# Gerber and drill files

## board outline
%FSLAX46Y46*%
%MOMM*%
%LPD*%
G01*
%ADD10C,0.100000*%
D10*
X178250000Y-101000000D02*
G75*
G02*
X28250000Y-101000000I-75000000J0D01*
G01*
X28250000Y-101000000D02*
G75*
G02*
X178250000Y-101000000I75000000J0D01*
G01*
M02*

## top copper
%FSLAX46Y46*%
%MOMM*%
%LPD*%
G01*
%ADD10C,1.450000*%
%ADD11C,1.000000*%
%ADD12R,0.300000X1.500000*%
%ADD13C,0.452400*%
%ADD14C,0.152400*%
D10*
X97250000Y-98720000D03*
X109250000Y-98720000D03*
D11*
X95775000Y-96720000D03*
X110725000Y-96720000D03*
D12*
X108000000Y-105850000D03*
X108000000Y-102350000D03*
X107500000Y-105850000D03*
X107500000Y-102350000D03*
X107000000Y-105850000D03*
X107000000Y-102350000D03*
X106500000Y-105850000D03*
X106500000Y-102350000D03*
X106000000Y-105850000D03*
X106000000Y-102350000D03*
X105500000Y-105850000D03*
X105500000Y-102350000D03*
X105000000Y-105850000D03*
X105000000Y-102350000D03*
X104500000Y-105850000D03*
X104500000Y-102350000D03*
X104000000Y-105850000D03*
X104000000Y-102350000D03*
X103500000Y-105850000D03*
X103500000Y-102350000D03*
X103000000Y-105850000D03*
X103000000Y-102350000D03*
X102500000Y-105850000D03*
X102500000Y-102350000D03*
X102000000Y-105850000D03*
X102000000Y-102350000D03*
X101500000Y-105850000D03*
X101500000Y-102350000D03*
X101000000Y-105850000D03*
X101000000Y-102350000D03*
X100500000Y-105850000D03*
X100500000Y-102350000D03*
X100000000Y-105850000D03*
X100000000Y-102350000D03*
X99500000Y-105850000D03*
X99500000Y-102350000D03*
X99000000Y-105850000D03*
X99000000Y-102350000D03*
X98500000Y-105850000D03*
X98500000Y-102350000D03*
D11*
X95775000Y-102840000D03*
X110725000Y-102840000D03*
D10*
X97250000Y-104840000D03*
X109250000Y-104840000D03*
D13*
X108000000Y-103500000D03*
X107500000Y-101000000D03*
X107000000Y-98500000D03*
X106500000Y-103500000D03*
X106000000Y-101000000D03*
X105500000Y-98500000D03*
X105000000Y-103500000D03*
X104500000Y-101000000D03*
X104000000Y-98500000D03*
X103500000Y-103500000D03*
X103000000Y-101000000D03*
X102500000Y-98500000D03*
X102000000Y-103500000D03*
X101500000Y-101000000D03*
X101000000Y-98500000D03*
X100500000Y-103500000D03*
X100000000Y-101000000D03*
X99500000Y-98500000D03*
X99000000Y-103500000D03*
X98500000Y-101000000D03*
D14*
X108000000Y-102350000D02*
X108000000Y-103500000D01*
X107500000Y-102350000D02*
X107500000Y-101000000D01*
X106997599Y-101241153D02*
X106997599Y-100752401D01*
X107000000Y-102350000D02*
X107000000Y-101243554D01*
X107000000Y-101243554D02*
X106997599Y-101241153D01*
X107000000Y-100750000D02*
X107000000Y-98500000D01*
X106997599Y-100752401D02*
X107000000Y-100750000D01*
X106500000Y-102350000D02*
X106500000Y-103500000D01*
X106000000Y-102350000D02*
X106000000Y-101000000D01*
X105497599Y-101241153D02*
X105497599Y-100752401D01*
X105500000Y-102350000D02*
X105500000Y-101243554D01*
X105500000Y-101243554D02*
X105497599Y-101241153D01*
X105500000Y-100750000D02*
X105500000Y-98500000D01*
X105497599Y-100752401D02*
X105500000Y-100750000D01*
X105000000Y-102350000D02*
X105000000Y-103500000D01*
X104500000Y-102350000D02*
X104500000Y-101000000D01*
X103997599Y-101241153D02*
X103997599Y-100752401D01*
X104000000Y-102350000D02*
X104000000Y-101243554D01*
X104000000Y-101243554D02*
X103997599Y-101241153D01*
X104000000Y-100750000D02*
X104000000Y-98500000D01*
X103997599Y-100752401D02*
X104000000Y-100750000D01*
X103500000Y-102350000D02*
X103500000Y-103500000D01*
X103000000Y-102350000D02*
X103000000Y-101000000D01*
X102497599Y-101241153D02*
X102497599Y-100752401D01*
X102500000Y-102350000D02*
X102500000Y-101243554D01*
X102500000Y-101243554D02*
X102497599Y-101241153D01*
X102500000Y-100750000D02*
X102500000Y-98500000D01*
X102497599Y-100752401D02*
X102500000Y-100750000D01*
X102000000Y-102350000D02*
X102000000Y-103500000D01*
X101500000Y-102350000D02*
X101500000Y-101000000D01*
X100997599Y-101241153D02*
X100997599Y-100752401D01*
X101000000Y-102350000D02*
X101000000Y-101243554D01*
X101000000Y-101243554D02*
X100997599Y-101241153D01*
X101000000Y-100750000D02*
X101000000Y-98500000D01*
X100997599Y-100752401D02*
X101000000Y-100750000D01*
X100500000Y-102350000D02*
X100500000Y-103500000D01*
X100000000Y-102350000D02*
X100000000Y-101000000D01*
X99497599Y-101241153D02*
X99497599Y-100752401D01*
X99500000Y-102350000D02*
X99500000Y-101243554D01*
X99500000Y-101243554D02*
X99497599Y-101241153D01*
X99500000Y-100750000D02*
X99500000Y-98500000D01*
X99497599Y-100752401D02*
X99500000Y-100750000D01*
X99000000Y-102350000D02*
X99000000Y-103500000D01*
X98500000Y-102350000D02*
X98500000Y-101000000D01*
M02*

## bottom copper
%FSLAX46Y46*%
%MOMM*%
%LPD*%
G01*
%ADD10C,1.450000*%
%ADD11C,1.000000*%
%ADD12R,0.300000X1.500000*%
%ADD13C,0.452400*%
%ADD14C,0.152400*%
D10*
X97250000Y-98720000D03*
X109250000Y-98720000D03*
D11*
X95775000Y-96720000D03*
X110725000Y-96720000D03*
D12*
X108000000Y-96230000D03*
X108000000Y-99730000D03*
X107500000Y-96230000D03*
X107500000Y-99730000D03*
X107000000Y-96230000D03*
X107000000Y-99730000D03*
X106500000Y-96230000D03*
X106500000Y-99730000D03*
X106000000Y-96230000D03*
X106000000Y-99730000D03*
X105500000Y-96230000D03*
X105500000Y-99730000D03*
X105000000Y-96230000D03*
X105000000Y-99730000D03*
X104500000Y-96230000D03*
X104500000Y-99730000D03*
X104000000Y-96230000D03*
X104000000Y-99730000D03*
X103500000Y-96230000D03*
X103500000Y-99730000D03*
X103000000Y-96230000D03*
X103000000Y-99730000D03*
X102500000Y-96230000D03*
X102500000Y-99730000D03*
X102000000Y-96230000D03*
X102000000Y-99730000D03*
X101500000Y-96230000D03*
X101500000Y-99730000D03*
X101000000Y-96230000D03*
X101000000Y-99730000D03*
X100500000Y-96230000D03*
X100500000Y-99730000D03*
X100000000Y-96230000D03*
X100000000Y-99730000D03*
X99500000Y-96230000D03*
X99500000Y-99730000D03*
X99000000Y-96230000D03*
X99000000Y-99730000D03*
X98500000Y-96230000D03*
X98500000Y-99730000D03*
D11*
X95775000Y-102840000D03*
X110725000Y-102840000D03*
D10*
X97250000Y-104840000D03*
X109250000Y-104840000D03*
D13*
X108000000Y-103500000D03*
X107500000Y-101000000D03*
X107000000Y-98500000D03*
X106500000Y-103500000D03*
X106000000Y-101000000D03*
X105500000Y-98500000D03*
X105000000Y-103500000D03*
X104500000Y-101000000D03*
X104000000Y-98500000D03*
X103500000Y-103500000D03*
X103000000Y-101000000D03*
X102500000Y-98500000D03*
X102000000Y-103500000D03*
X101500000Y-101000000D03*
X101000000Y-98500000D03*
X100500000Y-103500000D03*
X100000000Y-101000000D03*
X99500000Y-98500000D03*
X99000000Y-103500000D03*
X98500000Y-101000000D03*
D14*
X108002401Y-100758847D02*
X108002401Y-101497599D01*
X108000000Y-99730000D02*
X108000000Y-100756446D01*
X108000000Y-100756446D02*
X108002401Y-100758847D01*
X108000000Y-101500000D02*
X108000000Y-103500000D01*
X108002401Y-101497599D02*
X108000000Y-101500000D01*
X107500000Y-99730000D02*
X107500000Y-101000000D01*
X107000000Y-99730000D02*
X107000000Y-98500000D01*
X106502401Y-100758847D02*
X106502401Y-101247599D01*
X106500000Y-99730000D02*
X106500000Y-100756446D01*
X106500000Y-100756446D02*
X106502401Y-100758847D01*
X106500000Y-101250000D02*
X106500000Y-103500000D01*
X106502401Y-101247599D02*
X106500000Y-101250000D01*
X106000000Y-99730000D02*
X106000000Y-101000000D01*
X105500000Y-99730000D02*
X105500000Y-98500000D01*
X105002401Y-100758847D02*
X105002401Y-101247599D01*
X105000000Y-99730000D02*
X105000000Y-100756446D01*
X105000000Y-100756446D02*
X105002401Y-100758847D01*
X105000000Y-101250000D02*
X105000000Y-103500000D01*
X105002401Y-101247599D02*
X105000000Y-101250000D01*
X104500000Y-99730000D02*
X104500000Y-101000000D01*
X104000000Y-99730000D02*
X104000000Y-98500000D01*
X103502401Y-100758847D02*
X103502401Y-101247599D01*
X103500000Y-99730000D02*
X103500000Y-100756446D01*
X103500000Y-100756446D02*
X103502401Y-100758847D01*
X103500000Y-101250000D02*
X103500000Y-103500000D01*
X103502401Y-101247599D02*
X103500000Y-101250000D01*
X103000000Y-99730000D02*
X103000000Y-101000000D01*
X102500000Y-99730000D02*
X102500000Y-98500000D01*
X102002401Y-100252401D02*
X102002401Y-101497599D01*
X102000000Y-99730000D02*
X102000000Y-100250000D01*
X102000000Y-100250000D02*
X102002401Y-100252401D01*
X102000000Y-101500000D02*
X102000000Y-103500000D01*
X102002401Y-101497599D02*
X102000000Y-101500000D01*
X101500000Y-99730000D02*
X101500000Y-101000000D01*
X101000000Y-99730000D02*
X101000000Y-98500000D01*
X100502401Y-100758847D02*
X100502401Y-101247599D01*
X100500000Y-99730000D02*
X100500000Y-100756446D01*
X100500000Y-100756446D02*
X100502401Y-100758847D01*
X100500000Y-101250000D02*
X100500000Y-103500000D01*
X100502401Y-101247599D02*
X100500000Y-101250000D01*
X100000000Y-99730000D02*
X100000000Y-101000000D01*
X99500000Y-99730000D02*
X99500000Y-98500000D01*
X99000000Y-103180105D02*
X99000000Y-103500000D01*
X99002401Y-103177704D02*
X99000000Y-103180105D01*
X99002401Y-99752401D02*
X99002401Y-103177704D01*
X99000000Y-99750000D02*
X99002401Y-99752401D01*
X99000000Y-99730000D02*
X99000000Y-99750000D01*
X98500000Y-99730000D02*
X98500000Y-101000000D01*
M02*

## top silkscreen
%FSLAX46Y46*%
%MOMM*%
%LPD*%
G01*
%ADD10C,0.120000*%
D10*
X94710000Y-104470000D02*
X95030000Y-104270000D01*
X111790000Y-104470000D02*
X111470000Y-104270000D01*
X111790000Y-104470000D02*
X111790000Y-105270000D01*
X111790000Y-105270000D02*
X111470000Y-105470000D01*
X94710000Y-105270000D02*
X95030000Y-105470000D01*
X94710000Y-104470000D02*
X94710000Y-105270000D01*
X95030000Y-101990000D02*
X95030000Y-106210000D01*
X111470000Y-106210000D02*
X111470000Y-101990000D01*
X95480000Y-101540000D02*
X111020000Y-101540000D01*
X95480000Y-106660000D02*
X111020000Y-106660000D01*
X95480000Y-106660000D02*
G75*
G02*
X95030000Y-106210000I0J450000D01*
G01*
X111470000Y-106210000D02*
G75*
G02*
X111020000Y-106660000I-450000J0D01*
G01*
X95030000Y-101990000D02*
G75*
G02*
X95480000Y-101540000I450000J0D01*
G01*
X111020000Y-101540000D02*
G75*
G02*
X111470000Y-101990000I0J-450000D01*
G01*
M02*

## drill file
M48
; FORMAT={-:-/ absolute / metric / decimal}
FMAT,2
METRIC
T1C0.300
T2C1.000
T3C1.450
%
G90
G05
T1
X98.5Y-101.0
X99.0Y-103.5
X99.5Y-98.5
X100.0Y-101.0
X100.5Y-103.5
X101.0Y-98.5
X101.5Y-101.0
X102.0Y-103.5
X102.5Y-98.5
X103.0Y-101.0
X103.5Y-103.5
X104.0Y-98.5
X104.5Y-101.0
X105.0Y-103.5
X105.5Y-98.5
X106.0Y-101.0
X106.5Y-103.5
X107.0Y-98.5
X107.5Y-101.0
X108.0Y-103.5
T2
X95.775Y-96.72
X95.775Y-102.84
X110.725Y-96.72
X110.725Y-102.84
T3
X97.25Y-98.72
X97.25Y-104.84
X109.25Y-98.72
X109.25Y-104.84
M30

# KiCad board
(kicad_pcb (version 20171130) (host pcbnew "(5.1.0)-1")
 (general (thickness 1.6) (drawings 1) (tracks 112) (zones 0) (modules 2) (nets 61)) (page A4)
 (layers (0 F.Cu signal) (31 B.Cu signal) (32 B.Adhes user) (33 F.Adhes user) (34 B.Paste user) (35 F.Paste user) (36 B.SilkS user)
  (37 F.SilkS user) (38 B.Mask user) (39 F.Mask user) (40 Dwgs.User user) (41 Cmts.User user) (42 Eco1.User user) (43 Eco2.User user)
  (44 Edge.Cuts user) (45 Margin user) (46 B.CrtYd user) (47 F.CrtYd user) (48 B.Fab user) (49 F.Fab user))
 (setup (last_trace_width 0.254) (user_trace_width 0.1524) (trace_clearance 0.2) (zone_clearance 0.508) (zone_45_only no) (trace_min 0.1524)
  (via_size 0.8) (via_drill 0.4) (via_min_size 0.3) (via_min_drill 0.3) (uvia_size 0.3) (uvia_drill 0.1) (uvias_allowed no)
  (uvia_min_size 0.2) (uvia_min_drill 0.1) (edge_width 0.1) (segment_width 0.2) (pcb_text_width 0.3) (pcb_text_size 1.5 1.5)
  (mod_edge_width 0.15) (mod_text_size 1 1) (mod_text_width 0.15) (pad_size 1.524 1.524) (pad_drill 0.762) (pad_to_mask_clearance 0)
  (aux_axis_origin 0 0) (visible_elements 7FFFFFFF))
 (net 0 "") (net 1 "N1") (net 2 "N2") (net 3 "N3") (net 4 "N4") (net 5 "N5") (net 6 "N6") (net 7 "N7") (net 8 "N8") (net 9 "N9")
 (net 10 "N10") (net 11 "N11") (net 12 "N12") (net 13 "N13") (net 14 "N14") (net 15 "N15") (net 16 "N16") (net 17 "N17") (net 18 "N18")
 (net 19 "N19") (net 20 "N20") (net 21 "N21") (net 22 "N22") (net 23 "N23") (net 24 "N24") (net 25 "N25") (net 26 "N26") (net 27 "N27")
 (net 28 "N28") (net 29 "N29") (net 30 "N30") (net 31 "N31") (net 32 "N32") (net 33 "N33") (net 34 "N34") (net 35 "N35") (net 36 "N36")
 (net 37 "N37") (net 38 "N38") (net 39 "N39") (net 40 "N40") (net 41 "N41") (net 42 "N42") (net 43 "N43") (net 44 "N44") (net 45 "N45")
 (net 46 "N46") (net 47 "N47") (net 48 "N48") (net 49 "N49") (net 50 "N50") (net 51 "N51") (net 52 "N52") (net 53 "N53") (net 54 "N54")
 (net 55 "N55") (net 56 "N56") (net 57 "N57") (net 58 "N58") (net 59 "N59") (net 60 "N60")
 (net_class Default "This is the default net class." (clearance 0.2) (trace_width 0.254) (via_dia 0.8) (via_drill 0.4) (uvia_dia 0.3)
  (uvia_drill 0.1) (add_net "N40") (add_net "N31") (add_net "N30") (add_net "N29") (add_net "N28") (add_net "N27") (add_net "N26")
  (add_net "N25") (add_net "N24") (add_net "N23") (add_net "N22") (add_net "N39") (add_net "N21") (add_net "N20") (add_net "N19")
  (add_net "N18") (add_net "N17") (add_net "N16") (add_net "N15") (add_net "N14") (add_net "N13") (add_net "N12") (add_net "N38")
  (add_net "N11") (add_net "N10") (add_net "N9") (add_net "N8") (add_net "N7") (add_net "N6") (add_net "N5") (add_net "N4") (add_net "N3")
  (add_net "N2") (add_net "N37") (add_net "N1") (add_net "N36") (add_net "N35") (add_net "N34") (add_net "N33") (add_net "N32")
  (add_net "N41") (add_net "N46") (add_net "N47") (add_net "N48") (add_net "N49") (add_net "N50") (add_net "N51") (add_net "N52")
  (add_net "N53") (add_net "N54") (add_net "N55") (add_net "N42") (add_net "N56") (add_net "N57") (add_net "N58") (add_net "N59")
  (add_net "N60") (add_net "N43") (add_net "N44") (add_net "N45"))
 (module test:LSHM (layer B.Cu) (at 103.25 97.98 180)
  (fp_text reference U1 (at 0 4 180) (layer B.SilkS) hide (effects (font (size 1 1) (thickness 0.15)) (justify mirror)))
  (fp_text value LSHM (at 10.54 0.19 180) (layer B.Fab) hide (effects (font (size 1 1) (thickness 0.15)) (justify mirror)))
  (pad 41 thru_hole circle (at 6 -0.74 180) (size 1.45 1.45) (drill 1.45) (layers *.Cu *.Mask))
  (pad 41 thru_hole circle (at -6 -0.74 180) (size 1.45 1.45) (drill 1.45) (layers *.Cu *.Mask))
  (pad 41 thru_hole circle (at 7.475 1.26 180) (size 1 1) (drill 1) (layers *.Cu *.Mask))
  (pad 41 thru_hole circle (at -7.475 1.26 180) (size 1 1) (drill 1) (layers *.Cu *.Mask))
  (pad 40 smd rect (at -4.75 1.75 180) (size 0.3 1.5) (layers B.Cu B.Paste B.Mask) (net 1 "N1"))
  (pad 39 smd rect (at -4.75 -1.75 180) (size 0.3 1.5) (layers B.Cu B.Paste B.Mask) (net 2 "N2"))
  (pad 38 smd rect (at -4.25 1.75 180) (size 0.3 1.5) (layers B.Cu B.Paste B.Mask) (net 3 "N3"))
  (pad 37 smd rect (at -4.25 -1.75 180) (size 0.3 1.5) (layers B.Cu B.Paste B.Mask) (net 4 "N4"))
  (pad 36 smd rect (at -3.75 1.75 180) (size 0.3 1.5) (layers B.Cu B.Paste B.Mask) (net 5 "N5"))
  (pad 35 smd rect (at -3.75 -1.75 180) (size 0.3 1.5) (layers B.Cu B.Paste B.Mask) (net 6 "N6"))
  (pad 34 smd rect (at -3.25 1.75 180) (size 0.3 1.5) (layers B.Cu B.Paste B.Mask) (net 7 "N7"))
  (pad 33 smd rect (at -3.25 -1.75 180) (size 0.3 1.5) (layers B.Cu B.Paste B.Mask) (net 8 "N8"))
  (pad 32 smd rect (at -2.75 1.75 180) (size 0.3 1.5) (layers B.Cu B.Paste B.Mask) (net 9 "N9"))
  (pad 31 smd rect (at -2.75 -1.75 180) (size 0.3 1.5) (layers B.Cu B.Paste B.Mask) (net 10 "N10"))
  (pad 30 smd rect (at -2.25 1.75 180) (size 0.3 1.5) (layers B.Cu B.Paste B.Mask) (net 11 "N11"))
  (pad 29 smd rect (at -2.25 -1.75 180) (size 0.3 1.5) (layers B.Cu B.Paste B.Mask) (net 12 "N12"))
  (pad 28 smd rect (at -1.75 1.75 180) (size 0.3 1.5) (layers B.Cu B.Paste B.Mask) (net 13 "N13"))
  (pad 27 smd rect (at -1.75 -1.75 180) (size 0.3 1.5) (layers B.Cu B.Paste B.Mask) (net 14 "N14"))
  (pad 26 smd rect (at -1.25 1.75 180) (size 0.3 1.5) (layers B.Cu B.Paste B.Mask) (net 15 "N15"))
  (pad 25 smd rect (at -1.25 -1.75 180) (size 0.3 1.5) (layers B.Cu B.Paste B.Mask) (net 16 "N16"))
  (pad 24 smd rect (at -0.75 1.75 180) (size 0.3 1.5) (layers B.Cu B.Paste B.Mask) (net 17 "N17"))
  (pad 23 smd rect (at -0.75 -1.75 180) (size 0.3 1.5) (layers B.Cu B.Paste B.Mask) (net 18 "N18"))
  (pad 22 smd rect (at -0.25 1.75 180) (size 0.3 1.5) (layers B.Cu B.Paste B.Mask) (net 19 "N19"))
  (pad 21 smd rect (at -0.25 -1.75 180) (size 0.3 1.5) (layers B.Cu B.Paste B.Mask) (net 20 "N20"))
  (pad 20 smd rect (at 0.25 1.75 180) (size 0.3 1.5) (layers B.Cu B.Paste B.Mask) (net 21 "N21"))
  (pad 19 smd rect (at 0.25 -1.75 180) (size 0.3 1.5) (layers B.Cu B.Paste B.Mask) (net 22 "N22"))
  (pad 18 smd rect (at 0.75 1.75 180) (size 0.3 1.5) (layers B.Cu B.Paste B.Mask) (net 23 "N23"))
  (pad 17 smd rect (at 0.75 -1.75 180) (size 0.3 1.5) (layers B.Cu B.Paste B.Mask) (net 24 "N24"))
  (pad 16 smd rect (at 1.25 1.75 180) (size 0.3 1.5) (layers B.Cu B.Paste B.Mask) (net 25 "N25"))
  (pad 15 smd rect (at 1.25 -1.75 180) (size 0.3 1.5) (layers B.Cu B.Paste B.Mask) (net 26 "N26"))
  (pad 14 smd rect (at 1.75 1.75 180) (size 0.3 1.5) (layers B.Cu B.Paste B.Mask) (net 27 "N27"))
  (pad 13 smd rect (at 1.75 -1.75 180) (size 0.3 1.5) (layers B.Cu B.Paste B.Mask) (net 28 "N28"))
  (pad 12 smd rect (at 2.25 1.75 180) (size 0.3 1.5) (layers B.Cu B.Paste B.Mask) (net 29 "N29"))
  (pad 11 smd rect (at 2.25 -1.75 180) (size 0.3 1.5) (layers B.Cu B.Paste B.Mask) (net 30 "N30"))
  (pad 10 smd rect (at 2.75 1.75 180) (size 0.3 1.5) (layers B.Cu B.Paste B.Mask) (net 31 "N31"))
  (pad 9 smd rect (at 2.75 -1.75 180) (size 0.3 1.5) (layers B.Cu B.Paste B.Mask) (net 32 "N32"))
  (pad 8 smd rect (at 3.25 1.75 180) (size 0.3 1.5) (layers B.Cu B.Paste B.Mask) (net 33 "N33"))
  (pad 7 smd rect (at 3.25 -1.75 180) (size 0.3 1.5) (layers B.Cu B.Paste B.Mask) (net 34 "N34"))
  (pad 6 smd rect (at 3.75 1.75 180) (size 0.3 1.5) (layers B.Cu B.Paste B.Mask) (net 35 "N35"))
  (pad 5 smd rect (at 3.75 -1.75 180) (size 0.3 1.5) (layers B.Cu B.Paste B.Mask) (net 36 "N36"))
  (pad 4 smd rect (at 4.25 1.75 180) (size 0.3 1.5) (layers B.Cu B.Paste B.Mask) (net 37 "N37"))
  (pad 3 smd rect (at 4.25 -1.75 180) (size 0.3 1.5) (layers B.Cu B.Paste B.Mask) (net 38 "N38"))
  (pad 2 smd rect (at 4.75 1.75 180) (size 0.3 1.5) (layers B.Cu B.Paste B.Mask) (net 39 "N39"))
  (pad 1 smd rect (at 4.75 -1.75 180) (size 0.3 1.5) (layers B.Cu B.Paste B.Mask) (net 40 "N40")))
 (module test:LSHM (layer F.Cu) (at 103.25 104.1)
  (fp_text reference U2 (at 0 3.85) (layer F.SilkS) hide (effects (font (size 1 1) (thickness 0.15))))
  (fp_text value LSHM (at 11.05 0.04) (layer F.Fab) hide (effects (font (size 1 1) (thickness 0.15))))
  (fp_line (start -8.54 0.37) (end -8.22 0.17) (layer F.SilkS) (width 0.12))
  (fp_line (start 8.54 0.37) (end 8.22 0.17) (layer F.SilkS) (width 0.12))
  (fp_line (start 8.54 0.37) (end 8.54 1.17) (layer F.SilkS) (width 0.12))
  (fp_line (start 8.54 1.17) (end 8.22 1.37) (layer F.SilkS) (width 0.12))
  (fp_line (start -8.54 1.17) (end -8.22 1.37) (layer F.SilkS) (width 0.12))
  (fp_line (start -8.54 0.37) (end -8.54 1.17) (layer F.SilkS) (width 0.12))
  (fp_line (start -8.22 -2.11) (end -8.22 2.11) (layer F.SilkS) (width 0.12))
  (fp_line (start 8.22 2.11) (end 8.22 -2.11) (layer F.SilkS) (width 0.12))
  (fp_line (start -7.77 -2.56) (end 7.77 -2.56) (layer F.SilkS) (width 0.12))
  (fp_line (start -7.77 2.56) (end 7.77 2.56) (layer F.SilkS) (width 0.12))
  (fp_arc (start -7.77 2.11) (end -7.77 2.56) (angle 90) (layer F.SilkS) (width 0.12))
  (fp_arc (start 7.77 2.11) (end 8.22 2.11) (angle 90) (layer F.SilkS) (width 0.12))
  (fp_arc (start -7.77 -2.11) (end -8.22 -2.11) (angle 90) (layer F.SilkS) (width 0.12))
  (fp_arc (start 7.77 -2.11) (end 7.77 -2.56) (angle 90) (layer F.SilkS) (width 0.12))
  (pad 1 smd rect (at 4.75 1.75) (size 0.3 1.5) (layers F.Cu F.Paste F.Mask) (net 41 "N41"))
  (pad 2 smd rect (at 4.75 -1.75) (size 0.3 1.5) (layers F.Cu F.Paste F.Mask) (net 2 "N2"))
  (pad 3 smd rect (at 4.25 1.75) (size 0.3 1.5) (layers F.Cu F.Paste F.Mask) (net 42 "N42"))
  (pad 4 smd rect (at 4.25 -1.75) (size 0.3 1.5) (layers F.Cu F.Paste F.Mask) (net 4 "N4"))
  (pad 5 smd rect (at 3.75 1.75) (size 0.3 1.5) (layers F.Cu F.Paste F.Mask) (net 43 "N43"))
  (pad 6 smd rect (at 3.75 -1.75) (size 0.3 1.5) (layers F.Cu F.Paste F.Mask) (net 6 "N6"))
  (pad 7 smd rect (at 3.25 1.75) (size 0.3 1.5) (layers F.Cu F.Paste F.Mask) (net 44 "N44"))
  (pad 8 smd rect (at 3.25 -1.75) (size 0.3 1.5) (layers F.Cu F.Paste F.Mask) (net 8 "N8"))
  (pad 9 smd rect (at 2.75 1.75) (size 0.3 1.5) (layers F.Cu F.Paste F.Mask) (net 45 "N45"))
  (pad 10 smd rect (at 2.75 -1.75) (size 0.3 1.5) (layers F.Cu F.Paste F.Mask) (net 10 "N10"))
  (pad 11 smd rect (at 2.25 1.75) (size 0.3 1.5) (layers F.Cu F.Paste F.Mask) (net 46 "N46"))
  (pad 12 smd rect (at 2.25 -1.75) (size 0.3 1.5) (layers F.Cu F.Paste F.Mask) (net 12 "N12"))
  (pad 13 smd rect (at 1.75 1.75) (size 0.3 1.5) (layers F.Cu F.Paste F.Mask) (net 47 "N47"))
  (pad 14 smd rect (at 1.75 -1.75) (size 0.3 1.5) (layers F.Cu F.Paste F.Mask) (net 14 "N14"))
  (pad 15 smd rect (at 1.25 1.75) (size 0.3 1.5) (layers F.Cu F.Paste F.Mask) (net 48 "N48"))
  (pad 16 smd rect (at 1.25 -1.75) (size 0.3 1.5) (layers F.Cu F.Paste F.Mask) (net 16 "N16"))
  (pad 17 smd rect (at 0.75 1.75) (size 0.3 1.5) (layers F.Cu F.Paste F.Mask) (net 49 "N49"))
  (pad 18 smd rect (at 0.75 -1.75) (size 0.3 1.5) (layers F.Cu F.Paste F.Mask) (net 18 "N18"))
  (pad 19 smd rect (at 0.25 1.75) (size 0.3 1.5) (layers F.Cu F.Paste F.Mask) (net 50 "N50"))
  (pad 20 smd rect (at 0.25 -1.75) (size 0.3 1.5) (layers F.Cu F.Paste F.Mask) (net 20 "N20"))
  (pad 21 smd rect (at -0.25 1.75) (size 0.3 1.5) (layers F.Cu F.Paste F.Mask) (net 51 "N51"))
  (pad 22 smd rect (at -0.25 -1.75) (size 0.3 1.5) (layers F.Cu F.Paste F.Mask) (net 22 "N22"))
  (pad 23 smd rect (at -0.75 1.75) (size 0.3 1.5) (layers F.Cu F.Paste F.Mask) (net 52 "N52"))
  (pad 24 smd rect (at -0.75 -1.75) (size 0.3 1.5) (layers F.Cu F.Paste F.Mask) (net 24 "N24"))
  (pad 25 smd rect (at -1.25 1.75) (size 0.3 1.5) (layers F.Cu F.Paste F.Mask) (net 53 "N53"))
  (pad 26 smd rect (at -1.25 -1.75) (size 0.3 1.5) (layers F.Cu F.Paste F.Mask) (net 26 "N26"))
  (pad 27 smd rect (at -1.75 1.75) (size 0.3 1.5) (layers F.Cu F.Paste F.Mask) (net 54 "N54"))
  (pad 28 smd rect (at -1.75 -1.75) (size 0.3 1.5) (layers F.Cu F.Paste F.Mask) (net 28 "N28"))
  (pad 29 smd rect (at -2.25 1.75) (size 0.3 1.5) (layers F.Cu F.Paste F.Mask) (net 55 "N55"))
  (pad 30 smd rect (at -2.25 -1.75) (size 0.3 1.5) (layers F.Cu F.Paste F.Mask) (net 30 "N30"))
  (pad 31 smd rect (at -2.75 1.75) (size 0.3 1.5) (layers F.Cu F.Paste F.Mask) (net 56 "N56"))
  (pad 32 smd rect (at -2.75 -1.75) (size 0.3 1.5) (layers F.Cu F.Paste F.Mask) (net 32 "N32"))
  (pad 33 smd rect (at -3.25 1.75) (size 0.3 1.5) (layers F.Cu F.Paste F.Mask) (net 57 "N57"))
  (pad 34 smd rect (at -3.25 -1.75) (size 0.3 1.5) (layers F.Cu F.Paste F.Mask) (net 34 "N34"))
  (pad 35 smd rect (at -3.75 1.75) (size 0.3 1.5) (layers F.Cu F.Paste F.Mask) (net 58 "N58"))
  (pad 36 smd rect (at -3.75 -1.75) (size 0.3 1.5) (layers F.Cu F.Paste F.Mask) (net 36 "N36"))
  (pad 37 smd rect (at -4.25 1.75) (size 0.3 1.5) (layers F.Cu F.Paste F.Mask) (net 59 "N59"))
  (pad 38 smd rect (at -4.25 -1.75) (size 0.3 1.5) (layers F.Cu F.Paste F.Mask) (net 38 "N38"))
  (pad 39 smd rect (at -4.75 1.75) (size 0.3 1.5) (layers F.Cu F.Paste F.Mask) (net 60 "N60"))
  (pad 40 smd rect (at -4.75 -1.75) (size 0.3 1.5) (layers F.Cu F.Paste F.Mask) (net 40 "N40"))
  (pad 41 thru_hole circle (at -7.475 -1.26) (size 1 1) (drill 1) (layers *.Cu *.Mask))
  (pad 41 thru_hole circle (at 7.475 -1.26) (size 1 1) (drill 1) (layers *.Cu *.Mask))
  (pad 41 thru_hole circle (at -6 0.74) (size 1.45 1.45) (drill 1.45) (layers *.Cu *.Mask))
  (pad 41 thru_hole circle (at 6 0.74) (size 1.45 1.45) (drill 1.45) (layers *.Cu *.Mask)))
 (gr_circle (center 103.25 101) (end 178.25 101) (layer Edge.Cuts) (width 0.1))
 (via (at 108 103.5) (size 0.4524) (drill 0.3) (layers F.Cu B.Cu) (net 2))
 (segment (start 108 102.35) (end 108 103.5) (width 0.1524) (layer F.Cu) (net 2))
 (segment (start 108.002401 100.758847) (end 108.002401 101.497599) (width 0.1524) (layer B.Cu) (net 2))
 (segment (start 108 99.73) (end 108 100.756446) (width 0.1524) (layer B.Cu) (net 2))
 (segment (start 108 100.756446) (end 108.002401 100.758847) (width 0.1524) (layer B.Cu) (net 2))
 (segment (start 108 101.5) (end 108 103.5) (width 0.1524) (layer B.Cu) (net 2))
 (segment (start 108.002401 101.497599) (end 108 101.5) (width 0.1524) (layer B.Cu) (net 2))
 (via (at 107.5 101) (size 0.4524) (drill 0.3) (layers F.Cu B.Cu) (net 4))
 (segment (start 107.5 99.73) (end 107.5 101) (width 0.1524) (layer B.Cu) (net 4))
 (segment (start 107.5 102.35) (end 107.5 101) (width 0.1524) (layer F.Cu) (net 4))
 (via (at 107 98.5) (size 0.4524) (drill 0.3) (layers F.Cu B.Cu) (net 6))
 (segment (start 107 99.73) (end 107 98.5) (width 0.1524) (layer B.Cu) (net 6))
 (segment (start 106.997599 101.241153) (end 106.997599 100.752401) (width 0.1524) (layer F.Cu) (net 6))
 (segment (start 107 102.35) (end 107 101.243554) (width 0.1524) (layer F.Cu) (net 6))
 (segment (start 107 101.243554) (end 106.997599 101.241153) (width 0.1524) (layer F.Cu) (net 6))
 (segment (start 107 100.75) (end 107 98.5) (width 0.1524) (layer F.Cu) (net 6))
 (segment (start 106.997599 100.752401) (end 107 100.75) (width 0.1524) (layer F.Cu) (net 6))
 (via (at 106.5 103.5) (size 0.4524) (drill 0.3) (layers F.Cu B.Cu) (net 8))
 (segment (start 106.5 102.35) (end 106.5 103.5) (width 0.1524) (layer F.Cu) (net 8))
 (segment (start 106.502401 100.758847) (end 106.502401 101.247599) (width 0.1524) (layer B.Cu) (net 8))
 (segment (start 106.5 99.73) (end 106.5 100.756446) (width 0.1524) (layer B.Cu) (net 8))
 (segment (start 106.5 100.756446) (end 106.502401 100.758847) (width 0.1524) (layer B.Cu) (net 8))
 (segment (start 106.5 101.25) (end 106.5 103.5) (width 0.1524) (layer B.Cu) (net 8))
 (segment (start 106.502401 101.247599) (end 106.5 101.25) (width 0.1524) (layer B.Cu) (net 8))
 (via (at 106 101) (size 0.4524) (drill 0.3) (layers F.Cu B.Cu) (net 10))
 (segment (start 106 99.73) (end 106 101) (width 0.1524) (layer B.Cu) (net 10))
 (segment (start 106 102.35) (end 106 101) (width 0.1524) (layer F.Cu) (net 10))
 (via (at 105.5 98.5) (size 0.4524) (drill 0.3) (layers F.Cu B.Cu) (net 12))
 (segment (start 105.5 99.73) (end 105.5 98.5) (width 0.1524) (layer B.Cu) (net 12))
 (segment (start 105.497599 101.241153) (end 105.497599 100.752401) (width 0.1524) (layer F.Cu) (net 12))
 (segment (start 105.5 102.35) (end 105.5 101.243554) (width 0.1524) (layer F.Cu) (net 12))
 (segment (start 105.5 101.243554) (end 105.497599 101.241153) (width 0.1524) (layer F.Cu) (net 12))
 (segment (start 105.5 100.75) (end 105.5 98.5) (width 0.1524) (layer F.Cu) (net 12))
 (segment (start 105.497599 100.752401) (end 105.5 100.75) (width 0.1524) (layer F.Cu) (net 12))
 (via (at 105 103.5) (size 0.4524) (drill 0.3) (layers F.Cu B.Cu) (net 14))
 (segment (start 105 102.35) (end 105 103.5) (width 0.1524) (layer F.Cu) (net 14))
 (segment (start 105.002401 100.758847) (end 105.002401 101.247599) (width 0.1524) (layer B.Cu) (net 14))
 (segment (start 105 99.73) (end 105 100.756446) (width 0.1524) (layer B.Cu) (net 14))
 (segment (start 105 100.756446) (end 105.002401 100.758847) (width 0.1524) (layer B.Cu) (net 14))
 (segment (start 105 101.25) (end 105 103.5) (width 0.1524) (layer B.Cu) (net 14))
 (segment (start 105.002401 101.247599) (end 105 101.25) (width 0.1524) (layer B.Cu) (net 14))
 (via (at 104.5 101) (size 0.4524) (drill 0.3) (layers F.Cu B.Cu) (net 16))
 (segment (start 104.5 99.73) (end 104.5 101) (width 0.1524) (layer B.Cu) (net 16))
 (segment (start 104.5 102.35) (end 104.5 101) (width 0.1524) (layer F.Cu) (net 16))
 (via (at 104 98.5) (size 0.4524) (drill 0.3) (layers F.Cu B.Cu) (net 18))
 (segment (start 104 99.73) (end 104 98.5) (width 0.1524) (layer B.Cu) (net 18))
 (segment (start 103.997599 101.241153) (end 103.997599 100.752401) (width 0.1524) (layer F.Cu) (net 18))
 (segment (start 104 102.35) (end 104 101.243554) (width 0.1524) (layer F.Cu) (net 18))
 (segment (start 104 101.243554) (end 103.997599 101.241153) (width 0.1524) (layer F.Cu) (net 18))
 (segment (start 104 100.75) (end 104 98.5) (width 0.1524) (layer F.Cu) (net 18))
 (segment (start 103.997599 100.752401) (end 104 100.75) (width 0.1524) (layer F.Cu) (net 18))
 (via (at 103.5 103.5) (size 0.4524) (drill 0.3) (layers F.Cu B.Cu) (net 20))
 (segment (start 103.5 102.35) (end 103.5 103.5) (width 0.1524) (layer F.Cu) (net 20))
 (segment (start 103.502401 100.758847) (end 103.502401 101.247599) (width 0.1524) (layer B.Cu) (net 20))
 (segment (start 103.5 99.73) (end 103.5 100.756446) (width 0.1524) (layer B.Cu) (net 20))
 (segment (start 103.5 100.756446) (end 103.502401 100.758847) (width 0.1524) (layer B.Cu) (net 20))
 (segment (start 103.5 101.25) (end 103.5 103.5) (width 0.1524) (layer B.Cu) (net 20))
 (segment (start 103.502401 101.247599) (end 103.5 101.25) (width 0.1524) (layer B.Cu) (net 20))
 (via (at 103 101) (size 0.4524) (drill 0.3) (layers F.Cu B.Cu) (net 22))
 (segment (start 103 99.73) (end 103 101) (width 0.1524) (layer B.Cu) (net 22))
 (segment (start 103 102.35) (end 103 101) (width 0.1524) (layer F.Cu) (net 22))
 (via (at 102.5 98.5) (size 0.4524) (drill 0.3) (layers F.Cu B.Cu) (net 24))
 (segment (start 102.5 99.73) (end 102.5 98.5) (width 0.1524) (layer B.Cu) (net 24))
 (segment (start 102.497599 101.241153) (end 102.497599 100.752401) (width 0.1524) (layer F.Cu) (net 24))
 (segment (start 102.5 102.35) (end 102.5 101.243554) (width 0.1524) (layer F.Cu) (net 24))
 (segment (start 102.5 101.243554) (end 102.497599 101.241153) (width 0.1524) (layer F.Cu) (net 24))
 (segment (start 102.5 100.75) (end 102.5 98.5) (width 0.1524) (layer F.Cu) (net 24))
 (segment (start 102.497599 100.752401) (end 102.5 100.75) (width 0.1524) (layer F.Cu) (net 24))
 (via (at 102 103.5) (size 0.4524) (drill 0.3) (layers F.Cu B.Cu) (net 26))
 (segment (start 102 102.35) (end 102 103.5) (width 0.1524) (layer F.Cu) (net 26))
 (segment (start 102.002401 100.252401) (end 102.002401 101.497599) (width 0.1524) (layer B.Cu) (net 26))
 (segment (start 102 99.73) (end 102 100.25) (width 0.1524) (layer B.Cu) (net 26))
 (segment (start 102 100.25) (end 102.002401 100.252401) (width 0.1524) (layer B.Cu) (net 26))
 (segment (start 102 101.5) (end 102 103.5) (width 0.1524) (layer B.Cu) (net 26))
 (segment (start 102.002401 101.497599) (end 102 101.5) (width 0.1524) (layer B.Cu) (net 26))
 (via (at 101.5 101) (size 0.4524) (drill 0.3) (layers F.Cu B.Cu) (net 28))
 (segment (start 101.5 99.73) (end 101.5 101) (width 0.1524) (layer B.Cu) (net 28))
 (segment (start 101.5 102.35) (end 101.5 101) (width 0.1524) (layer F.Cu) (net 28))
 (via (at 101 98.5) (size 0.4524) (drill 0.3) (layers F.Cu B.Cu) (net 30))
 (segment (start 101 99.73) (end 101 98.5) (width 0.1524) (layer B.Cu) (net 30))
 (segment (start 100.997599 101.241153) (end 100.997599 100.752401) (width 0.1524) (layer F.Cu) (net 30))
 (segment (start 101 102.35) (end 101 101.243554) (width 0.1524) (layer F.Cu) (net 30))
 (segment (start 101 101.243554) (end 100.997599 101.241153) (width 0.1524) (layer F.Cu) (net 30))
 (segment (start 101 100.75) (end 101 98.5) (width 0.1524) (layer F.Cu) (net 30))
 (segment (start 100.997599 100.752401) (end 101 100.75) (width 0.1524) (layer F.Cu) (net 30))
 (via (at 100.5 103.5) (size 0.4524) (drill 0.3) (layers F.Cu B.Cu) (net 32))
 (segment (start 100.502401 100.758847) (end 100.502401 101.247599) (width 0.1524) (layer B.Cu) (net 32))
 (segment (start 100.5 99.73) (end 100.5 100.756446) (width 0.1524) (layer B.Cu) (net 32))
 (segment (start 100.5 100.756446) (end 100.502401 100.758847) (width 0.1524) (layer B.Cu) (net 32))
 (segment (start 100.5 102.35) (end 100.5 103.5) (width 0.1524) (layer F.Cu) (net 32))
 (segment (start 100.5 101.25) (end 100.5 103.5) (width 0.1524) (layer B.Cu) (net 32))
 (segment (start 100.502401 101.247599) (end 100.5 101.25) (width 0.1524) (layer B.Cu) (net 32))
 (via (at 100 101) (size 0.4524) (drill 0.3) (layers F.Cu B.Cu) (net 34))
 (segment (start 100 99.73) (end 100 101) (width 0.1524) (layer B.Cu) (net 34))
 (segment (start 100 102.35) (end 100 101) (width 0.1524) (layer F.Cu) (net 34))
 (via (at 99.5 98.5) (size 0.4524) (drill 0.3) (layers F.Cu B.Cu) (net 36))
 (segment (start 99.5 99.73) (end 99.5 98.5) (width 0.1524) (layer B.Cu) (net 36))
 (segment (start 99.497599 101.241153) (end 99.497599 100.752401) (width 0.1524) (layer F.Cu) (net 36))
 (segment (start 99.5 102.35) (end 99.5 101.243554) (width 0.1524) (layer F.Cu) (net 36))
 (segment (start 99.5 101.243554) (end 99.497599 101.241153) (width 0.1524) (layer F.Cu) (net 36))
 (segment (start 99.5 100.75) (end 99.5 98.5) (width 0.1524) (layer F.Cu) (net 36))
 (segment (start 99.497599 100.752401) (end 99.5 100.75) (width 0.1524) (layer F.Cu) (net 36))
 (via (at 99 103.5) (size 0.4524) (drill 0.3) (layers F.Cu B.Cu) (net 38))
 (segment (start 99 102.35) (end 99 103.5) (width 0.1524) (layer F.Cu) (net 38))
 (segment (start 99 103.180105) (end 99 103.5) (width 0.1524) (layer B.Cu) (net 38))
 (segment (start 99.002401 103.177704) (end 99 103.180105) (width 0.1524) (layer B.Cu) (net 38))
 (segment (start 99.002401 99.752401) (end 99.002401 103.177704) (width 0.1524) (layer B.Cu) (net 38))
 (segment (start 99 99.75) (end 99.002401 99.752401) (width 0.1524) (layer B.Cu) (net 38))
 (segment (start 99 99.73) (end 99 99.75) (width 0.1524) (layer B.Cu) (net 38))
 (via (at 98.5 101) (size 0.4524) (drill 0.3) (layers F.Cu B.Cu) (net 40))
 (segment (start 98.5 99.73) (end 98.5 101) (width 0.1524) (layer B.Cu) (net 40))
 (segment (start 98.5 102.35) (end 98.5 101) (width 0.1524) (layer F.Cu) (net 40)))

